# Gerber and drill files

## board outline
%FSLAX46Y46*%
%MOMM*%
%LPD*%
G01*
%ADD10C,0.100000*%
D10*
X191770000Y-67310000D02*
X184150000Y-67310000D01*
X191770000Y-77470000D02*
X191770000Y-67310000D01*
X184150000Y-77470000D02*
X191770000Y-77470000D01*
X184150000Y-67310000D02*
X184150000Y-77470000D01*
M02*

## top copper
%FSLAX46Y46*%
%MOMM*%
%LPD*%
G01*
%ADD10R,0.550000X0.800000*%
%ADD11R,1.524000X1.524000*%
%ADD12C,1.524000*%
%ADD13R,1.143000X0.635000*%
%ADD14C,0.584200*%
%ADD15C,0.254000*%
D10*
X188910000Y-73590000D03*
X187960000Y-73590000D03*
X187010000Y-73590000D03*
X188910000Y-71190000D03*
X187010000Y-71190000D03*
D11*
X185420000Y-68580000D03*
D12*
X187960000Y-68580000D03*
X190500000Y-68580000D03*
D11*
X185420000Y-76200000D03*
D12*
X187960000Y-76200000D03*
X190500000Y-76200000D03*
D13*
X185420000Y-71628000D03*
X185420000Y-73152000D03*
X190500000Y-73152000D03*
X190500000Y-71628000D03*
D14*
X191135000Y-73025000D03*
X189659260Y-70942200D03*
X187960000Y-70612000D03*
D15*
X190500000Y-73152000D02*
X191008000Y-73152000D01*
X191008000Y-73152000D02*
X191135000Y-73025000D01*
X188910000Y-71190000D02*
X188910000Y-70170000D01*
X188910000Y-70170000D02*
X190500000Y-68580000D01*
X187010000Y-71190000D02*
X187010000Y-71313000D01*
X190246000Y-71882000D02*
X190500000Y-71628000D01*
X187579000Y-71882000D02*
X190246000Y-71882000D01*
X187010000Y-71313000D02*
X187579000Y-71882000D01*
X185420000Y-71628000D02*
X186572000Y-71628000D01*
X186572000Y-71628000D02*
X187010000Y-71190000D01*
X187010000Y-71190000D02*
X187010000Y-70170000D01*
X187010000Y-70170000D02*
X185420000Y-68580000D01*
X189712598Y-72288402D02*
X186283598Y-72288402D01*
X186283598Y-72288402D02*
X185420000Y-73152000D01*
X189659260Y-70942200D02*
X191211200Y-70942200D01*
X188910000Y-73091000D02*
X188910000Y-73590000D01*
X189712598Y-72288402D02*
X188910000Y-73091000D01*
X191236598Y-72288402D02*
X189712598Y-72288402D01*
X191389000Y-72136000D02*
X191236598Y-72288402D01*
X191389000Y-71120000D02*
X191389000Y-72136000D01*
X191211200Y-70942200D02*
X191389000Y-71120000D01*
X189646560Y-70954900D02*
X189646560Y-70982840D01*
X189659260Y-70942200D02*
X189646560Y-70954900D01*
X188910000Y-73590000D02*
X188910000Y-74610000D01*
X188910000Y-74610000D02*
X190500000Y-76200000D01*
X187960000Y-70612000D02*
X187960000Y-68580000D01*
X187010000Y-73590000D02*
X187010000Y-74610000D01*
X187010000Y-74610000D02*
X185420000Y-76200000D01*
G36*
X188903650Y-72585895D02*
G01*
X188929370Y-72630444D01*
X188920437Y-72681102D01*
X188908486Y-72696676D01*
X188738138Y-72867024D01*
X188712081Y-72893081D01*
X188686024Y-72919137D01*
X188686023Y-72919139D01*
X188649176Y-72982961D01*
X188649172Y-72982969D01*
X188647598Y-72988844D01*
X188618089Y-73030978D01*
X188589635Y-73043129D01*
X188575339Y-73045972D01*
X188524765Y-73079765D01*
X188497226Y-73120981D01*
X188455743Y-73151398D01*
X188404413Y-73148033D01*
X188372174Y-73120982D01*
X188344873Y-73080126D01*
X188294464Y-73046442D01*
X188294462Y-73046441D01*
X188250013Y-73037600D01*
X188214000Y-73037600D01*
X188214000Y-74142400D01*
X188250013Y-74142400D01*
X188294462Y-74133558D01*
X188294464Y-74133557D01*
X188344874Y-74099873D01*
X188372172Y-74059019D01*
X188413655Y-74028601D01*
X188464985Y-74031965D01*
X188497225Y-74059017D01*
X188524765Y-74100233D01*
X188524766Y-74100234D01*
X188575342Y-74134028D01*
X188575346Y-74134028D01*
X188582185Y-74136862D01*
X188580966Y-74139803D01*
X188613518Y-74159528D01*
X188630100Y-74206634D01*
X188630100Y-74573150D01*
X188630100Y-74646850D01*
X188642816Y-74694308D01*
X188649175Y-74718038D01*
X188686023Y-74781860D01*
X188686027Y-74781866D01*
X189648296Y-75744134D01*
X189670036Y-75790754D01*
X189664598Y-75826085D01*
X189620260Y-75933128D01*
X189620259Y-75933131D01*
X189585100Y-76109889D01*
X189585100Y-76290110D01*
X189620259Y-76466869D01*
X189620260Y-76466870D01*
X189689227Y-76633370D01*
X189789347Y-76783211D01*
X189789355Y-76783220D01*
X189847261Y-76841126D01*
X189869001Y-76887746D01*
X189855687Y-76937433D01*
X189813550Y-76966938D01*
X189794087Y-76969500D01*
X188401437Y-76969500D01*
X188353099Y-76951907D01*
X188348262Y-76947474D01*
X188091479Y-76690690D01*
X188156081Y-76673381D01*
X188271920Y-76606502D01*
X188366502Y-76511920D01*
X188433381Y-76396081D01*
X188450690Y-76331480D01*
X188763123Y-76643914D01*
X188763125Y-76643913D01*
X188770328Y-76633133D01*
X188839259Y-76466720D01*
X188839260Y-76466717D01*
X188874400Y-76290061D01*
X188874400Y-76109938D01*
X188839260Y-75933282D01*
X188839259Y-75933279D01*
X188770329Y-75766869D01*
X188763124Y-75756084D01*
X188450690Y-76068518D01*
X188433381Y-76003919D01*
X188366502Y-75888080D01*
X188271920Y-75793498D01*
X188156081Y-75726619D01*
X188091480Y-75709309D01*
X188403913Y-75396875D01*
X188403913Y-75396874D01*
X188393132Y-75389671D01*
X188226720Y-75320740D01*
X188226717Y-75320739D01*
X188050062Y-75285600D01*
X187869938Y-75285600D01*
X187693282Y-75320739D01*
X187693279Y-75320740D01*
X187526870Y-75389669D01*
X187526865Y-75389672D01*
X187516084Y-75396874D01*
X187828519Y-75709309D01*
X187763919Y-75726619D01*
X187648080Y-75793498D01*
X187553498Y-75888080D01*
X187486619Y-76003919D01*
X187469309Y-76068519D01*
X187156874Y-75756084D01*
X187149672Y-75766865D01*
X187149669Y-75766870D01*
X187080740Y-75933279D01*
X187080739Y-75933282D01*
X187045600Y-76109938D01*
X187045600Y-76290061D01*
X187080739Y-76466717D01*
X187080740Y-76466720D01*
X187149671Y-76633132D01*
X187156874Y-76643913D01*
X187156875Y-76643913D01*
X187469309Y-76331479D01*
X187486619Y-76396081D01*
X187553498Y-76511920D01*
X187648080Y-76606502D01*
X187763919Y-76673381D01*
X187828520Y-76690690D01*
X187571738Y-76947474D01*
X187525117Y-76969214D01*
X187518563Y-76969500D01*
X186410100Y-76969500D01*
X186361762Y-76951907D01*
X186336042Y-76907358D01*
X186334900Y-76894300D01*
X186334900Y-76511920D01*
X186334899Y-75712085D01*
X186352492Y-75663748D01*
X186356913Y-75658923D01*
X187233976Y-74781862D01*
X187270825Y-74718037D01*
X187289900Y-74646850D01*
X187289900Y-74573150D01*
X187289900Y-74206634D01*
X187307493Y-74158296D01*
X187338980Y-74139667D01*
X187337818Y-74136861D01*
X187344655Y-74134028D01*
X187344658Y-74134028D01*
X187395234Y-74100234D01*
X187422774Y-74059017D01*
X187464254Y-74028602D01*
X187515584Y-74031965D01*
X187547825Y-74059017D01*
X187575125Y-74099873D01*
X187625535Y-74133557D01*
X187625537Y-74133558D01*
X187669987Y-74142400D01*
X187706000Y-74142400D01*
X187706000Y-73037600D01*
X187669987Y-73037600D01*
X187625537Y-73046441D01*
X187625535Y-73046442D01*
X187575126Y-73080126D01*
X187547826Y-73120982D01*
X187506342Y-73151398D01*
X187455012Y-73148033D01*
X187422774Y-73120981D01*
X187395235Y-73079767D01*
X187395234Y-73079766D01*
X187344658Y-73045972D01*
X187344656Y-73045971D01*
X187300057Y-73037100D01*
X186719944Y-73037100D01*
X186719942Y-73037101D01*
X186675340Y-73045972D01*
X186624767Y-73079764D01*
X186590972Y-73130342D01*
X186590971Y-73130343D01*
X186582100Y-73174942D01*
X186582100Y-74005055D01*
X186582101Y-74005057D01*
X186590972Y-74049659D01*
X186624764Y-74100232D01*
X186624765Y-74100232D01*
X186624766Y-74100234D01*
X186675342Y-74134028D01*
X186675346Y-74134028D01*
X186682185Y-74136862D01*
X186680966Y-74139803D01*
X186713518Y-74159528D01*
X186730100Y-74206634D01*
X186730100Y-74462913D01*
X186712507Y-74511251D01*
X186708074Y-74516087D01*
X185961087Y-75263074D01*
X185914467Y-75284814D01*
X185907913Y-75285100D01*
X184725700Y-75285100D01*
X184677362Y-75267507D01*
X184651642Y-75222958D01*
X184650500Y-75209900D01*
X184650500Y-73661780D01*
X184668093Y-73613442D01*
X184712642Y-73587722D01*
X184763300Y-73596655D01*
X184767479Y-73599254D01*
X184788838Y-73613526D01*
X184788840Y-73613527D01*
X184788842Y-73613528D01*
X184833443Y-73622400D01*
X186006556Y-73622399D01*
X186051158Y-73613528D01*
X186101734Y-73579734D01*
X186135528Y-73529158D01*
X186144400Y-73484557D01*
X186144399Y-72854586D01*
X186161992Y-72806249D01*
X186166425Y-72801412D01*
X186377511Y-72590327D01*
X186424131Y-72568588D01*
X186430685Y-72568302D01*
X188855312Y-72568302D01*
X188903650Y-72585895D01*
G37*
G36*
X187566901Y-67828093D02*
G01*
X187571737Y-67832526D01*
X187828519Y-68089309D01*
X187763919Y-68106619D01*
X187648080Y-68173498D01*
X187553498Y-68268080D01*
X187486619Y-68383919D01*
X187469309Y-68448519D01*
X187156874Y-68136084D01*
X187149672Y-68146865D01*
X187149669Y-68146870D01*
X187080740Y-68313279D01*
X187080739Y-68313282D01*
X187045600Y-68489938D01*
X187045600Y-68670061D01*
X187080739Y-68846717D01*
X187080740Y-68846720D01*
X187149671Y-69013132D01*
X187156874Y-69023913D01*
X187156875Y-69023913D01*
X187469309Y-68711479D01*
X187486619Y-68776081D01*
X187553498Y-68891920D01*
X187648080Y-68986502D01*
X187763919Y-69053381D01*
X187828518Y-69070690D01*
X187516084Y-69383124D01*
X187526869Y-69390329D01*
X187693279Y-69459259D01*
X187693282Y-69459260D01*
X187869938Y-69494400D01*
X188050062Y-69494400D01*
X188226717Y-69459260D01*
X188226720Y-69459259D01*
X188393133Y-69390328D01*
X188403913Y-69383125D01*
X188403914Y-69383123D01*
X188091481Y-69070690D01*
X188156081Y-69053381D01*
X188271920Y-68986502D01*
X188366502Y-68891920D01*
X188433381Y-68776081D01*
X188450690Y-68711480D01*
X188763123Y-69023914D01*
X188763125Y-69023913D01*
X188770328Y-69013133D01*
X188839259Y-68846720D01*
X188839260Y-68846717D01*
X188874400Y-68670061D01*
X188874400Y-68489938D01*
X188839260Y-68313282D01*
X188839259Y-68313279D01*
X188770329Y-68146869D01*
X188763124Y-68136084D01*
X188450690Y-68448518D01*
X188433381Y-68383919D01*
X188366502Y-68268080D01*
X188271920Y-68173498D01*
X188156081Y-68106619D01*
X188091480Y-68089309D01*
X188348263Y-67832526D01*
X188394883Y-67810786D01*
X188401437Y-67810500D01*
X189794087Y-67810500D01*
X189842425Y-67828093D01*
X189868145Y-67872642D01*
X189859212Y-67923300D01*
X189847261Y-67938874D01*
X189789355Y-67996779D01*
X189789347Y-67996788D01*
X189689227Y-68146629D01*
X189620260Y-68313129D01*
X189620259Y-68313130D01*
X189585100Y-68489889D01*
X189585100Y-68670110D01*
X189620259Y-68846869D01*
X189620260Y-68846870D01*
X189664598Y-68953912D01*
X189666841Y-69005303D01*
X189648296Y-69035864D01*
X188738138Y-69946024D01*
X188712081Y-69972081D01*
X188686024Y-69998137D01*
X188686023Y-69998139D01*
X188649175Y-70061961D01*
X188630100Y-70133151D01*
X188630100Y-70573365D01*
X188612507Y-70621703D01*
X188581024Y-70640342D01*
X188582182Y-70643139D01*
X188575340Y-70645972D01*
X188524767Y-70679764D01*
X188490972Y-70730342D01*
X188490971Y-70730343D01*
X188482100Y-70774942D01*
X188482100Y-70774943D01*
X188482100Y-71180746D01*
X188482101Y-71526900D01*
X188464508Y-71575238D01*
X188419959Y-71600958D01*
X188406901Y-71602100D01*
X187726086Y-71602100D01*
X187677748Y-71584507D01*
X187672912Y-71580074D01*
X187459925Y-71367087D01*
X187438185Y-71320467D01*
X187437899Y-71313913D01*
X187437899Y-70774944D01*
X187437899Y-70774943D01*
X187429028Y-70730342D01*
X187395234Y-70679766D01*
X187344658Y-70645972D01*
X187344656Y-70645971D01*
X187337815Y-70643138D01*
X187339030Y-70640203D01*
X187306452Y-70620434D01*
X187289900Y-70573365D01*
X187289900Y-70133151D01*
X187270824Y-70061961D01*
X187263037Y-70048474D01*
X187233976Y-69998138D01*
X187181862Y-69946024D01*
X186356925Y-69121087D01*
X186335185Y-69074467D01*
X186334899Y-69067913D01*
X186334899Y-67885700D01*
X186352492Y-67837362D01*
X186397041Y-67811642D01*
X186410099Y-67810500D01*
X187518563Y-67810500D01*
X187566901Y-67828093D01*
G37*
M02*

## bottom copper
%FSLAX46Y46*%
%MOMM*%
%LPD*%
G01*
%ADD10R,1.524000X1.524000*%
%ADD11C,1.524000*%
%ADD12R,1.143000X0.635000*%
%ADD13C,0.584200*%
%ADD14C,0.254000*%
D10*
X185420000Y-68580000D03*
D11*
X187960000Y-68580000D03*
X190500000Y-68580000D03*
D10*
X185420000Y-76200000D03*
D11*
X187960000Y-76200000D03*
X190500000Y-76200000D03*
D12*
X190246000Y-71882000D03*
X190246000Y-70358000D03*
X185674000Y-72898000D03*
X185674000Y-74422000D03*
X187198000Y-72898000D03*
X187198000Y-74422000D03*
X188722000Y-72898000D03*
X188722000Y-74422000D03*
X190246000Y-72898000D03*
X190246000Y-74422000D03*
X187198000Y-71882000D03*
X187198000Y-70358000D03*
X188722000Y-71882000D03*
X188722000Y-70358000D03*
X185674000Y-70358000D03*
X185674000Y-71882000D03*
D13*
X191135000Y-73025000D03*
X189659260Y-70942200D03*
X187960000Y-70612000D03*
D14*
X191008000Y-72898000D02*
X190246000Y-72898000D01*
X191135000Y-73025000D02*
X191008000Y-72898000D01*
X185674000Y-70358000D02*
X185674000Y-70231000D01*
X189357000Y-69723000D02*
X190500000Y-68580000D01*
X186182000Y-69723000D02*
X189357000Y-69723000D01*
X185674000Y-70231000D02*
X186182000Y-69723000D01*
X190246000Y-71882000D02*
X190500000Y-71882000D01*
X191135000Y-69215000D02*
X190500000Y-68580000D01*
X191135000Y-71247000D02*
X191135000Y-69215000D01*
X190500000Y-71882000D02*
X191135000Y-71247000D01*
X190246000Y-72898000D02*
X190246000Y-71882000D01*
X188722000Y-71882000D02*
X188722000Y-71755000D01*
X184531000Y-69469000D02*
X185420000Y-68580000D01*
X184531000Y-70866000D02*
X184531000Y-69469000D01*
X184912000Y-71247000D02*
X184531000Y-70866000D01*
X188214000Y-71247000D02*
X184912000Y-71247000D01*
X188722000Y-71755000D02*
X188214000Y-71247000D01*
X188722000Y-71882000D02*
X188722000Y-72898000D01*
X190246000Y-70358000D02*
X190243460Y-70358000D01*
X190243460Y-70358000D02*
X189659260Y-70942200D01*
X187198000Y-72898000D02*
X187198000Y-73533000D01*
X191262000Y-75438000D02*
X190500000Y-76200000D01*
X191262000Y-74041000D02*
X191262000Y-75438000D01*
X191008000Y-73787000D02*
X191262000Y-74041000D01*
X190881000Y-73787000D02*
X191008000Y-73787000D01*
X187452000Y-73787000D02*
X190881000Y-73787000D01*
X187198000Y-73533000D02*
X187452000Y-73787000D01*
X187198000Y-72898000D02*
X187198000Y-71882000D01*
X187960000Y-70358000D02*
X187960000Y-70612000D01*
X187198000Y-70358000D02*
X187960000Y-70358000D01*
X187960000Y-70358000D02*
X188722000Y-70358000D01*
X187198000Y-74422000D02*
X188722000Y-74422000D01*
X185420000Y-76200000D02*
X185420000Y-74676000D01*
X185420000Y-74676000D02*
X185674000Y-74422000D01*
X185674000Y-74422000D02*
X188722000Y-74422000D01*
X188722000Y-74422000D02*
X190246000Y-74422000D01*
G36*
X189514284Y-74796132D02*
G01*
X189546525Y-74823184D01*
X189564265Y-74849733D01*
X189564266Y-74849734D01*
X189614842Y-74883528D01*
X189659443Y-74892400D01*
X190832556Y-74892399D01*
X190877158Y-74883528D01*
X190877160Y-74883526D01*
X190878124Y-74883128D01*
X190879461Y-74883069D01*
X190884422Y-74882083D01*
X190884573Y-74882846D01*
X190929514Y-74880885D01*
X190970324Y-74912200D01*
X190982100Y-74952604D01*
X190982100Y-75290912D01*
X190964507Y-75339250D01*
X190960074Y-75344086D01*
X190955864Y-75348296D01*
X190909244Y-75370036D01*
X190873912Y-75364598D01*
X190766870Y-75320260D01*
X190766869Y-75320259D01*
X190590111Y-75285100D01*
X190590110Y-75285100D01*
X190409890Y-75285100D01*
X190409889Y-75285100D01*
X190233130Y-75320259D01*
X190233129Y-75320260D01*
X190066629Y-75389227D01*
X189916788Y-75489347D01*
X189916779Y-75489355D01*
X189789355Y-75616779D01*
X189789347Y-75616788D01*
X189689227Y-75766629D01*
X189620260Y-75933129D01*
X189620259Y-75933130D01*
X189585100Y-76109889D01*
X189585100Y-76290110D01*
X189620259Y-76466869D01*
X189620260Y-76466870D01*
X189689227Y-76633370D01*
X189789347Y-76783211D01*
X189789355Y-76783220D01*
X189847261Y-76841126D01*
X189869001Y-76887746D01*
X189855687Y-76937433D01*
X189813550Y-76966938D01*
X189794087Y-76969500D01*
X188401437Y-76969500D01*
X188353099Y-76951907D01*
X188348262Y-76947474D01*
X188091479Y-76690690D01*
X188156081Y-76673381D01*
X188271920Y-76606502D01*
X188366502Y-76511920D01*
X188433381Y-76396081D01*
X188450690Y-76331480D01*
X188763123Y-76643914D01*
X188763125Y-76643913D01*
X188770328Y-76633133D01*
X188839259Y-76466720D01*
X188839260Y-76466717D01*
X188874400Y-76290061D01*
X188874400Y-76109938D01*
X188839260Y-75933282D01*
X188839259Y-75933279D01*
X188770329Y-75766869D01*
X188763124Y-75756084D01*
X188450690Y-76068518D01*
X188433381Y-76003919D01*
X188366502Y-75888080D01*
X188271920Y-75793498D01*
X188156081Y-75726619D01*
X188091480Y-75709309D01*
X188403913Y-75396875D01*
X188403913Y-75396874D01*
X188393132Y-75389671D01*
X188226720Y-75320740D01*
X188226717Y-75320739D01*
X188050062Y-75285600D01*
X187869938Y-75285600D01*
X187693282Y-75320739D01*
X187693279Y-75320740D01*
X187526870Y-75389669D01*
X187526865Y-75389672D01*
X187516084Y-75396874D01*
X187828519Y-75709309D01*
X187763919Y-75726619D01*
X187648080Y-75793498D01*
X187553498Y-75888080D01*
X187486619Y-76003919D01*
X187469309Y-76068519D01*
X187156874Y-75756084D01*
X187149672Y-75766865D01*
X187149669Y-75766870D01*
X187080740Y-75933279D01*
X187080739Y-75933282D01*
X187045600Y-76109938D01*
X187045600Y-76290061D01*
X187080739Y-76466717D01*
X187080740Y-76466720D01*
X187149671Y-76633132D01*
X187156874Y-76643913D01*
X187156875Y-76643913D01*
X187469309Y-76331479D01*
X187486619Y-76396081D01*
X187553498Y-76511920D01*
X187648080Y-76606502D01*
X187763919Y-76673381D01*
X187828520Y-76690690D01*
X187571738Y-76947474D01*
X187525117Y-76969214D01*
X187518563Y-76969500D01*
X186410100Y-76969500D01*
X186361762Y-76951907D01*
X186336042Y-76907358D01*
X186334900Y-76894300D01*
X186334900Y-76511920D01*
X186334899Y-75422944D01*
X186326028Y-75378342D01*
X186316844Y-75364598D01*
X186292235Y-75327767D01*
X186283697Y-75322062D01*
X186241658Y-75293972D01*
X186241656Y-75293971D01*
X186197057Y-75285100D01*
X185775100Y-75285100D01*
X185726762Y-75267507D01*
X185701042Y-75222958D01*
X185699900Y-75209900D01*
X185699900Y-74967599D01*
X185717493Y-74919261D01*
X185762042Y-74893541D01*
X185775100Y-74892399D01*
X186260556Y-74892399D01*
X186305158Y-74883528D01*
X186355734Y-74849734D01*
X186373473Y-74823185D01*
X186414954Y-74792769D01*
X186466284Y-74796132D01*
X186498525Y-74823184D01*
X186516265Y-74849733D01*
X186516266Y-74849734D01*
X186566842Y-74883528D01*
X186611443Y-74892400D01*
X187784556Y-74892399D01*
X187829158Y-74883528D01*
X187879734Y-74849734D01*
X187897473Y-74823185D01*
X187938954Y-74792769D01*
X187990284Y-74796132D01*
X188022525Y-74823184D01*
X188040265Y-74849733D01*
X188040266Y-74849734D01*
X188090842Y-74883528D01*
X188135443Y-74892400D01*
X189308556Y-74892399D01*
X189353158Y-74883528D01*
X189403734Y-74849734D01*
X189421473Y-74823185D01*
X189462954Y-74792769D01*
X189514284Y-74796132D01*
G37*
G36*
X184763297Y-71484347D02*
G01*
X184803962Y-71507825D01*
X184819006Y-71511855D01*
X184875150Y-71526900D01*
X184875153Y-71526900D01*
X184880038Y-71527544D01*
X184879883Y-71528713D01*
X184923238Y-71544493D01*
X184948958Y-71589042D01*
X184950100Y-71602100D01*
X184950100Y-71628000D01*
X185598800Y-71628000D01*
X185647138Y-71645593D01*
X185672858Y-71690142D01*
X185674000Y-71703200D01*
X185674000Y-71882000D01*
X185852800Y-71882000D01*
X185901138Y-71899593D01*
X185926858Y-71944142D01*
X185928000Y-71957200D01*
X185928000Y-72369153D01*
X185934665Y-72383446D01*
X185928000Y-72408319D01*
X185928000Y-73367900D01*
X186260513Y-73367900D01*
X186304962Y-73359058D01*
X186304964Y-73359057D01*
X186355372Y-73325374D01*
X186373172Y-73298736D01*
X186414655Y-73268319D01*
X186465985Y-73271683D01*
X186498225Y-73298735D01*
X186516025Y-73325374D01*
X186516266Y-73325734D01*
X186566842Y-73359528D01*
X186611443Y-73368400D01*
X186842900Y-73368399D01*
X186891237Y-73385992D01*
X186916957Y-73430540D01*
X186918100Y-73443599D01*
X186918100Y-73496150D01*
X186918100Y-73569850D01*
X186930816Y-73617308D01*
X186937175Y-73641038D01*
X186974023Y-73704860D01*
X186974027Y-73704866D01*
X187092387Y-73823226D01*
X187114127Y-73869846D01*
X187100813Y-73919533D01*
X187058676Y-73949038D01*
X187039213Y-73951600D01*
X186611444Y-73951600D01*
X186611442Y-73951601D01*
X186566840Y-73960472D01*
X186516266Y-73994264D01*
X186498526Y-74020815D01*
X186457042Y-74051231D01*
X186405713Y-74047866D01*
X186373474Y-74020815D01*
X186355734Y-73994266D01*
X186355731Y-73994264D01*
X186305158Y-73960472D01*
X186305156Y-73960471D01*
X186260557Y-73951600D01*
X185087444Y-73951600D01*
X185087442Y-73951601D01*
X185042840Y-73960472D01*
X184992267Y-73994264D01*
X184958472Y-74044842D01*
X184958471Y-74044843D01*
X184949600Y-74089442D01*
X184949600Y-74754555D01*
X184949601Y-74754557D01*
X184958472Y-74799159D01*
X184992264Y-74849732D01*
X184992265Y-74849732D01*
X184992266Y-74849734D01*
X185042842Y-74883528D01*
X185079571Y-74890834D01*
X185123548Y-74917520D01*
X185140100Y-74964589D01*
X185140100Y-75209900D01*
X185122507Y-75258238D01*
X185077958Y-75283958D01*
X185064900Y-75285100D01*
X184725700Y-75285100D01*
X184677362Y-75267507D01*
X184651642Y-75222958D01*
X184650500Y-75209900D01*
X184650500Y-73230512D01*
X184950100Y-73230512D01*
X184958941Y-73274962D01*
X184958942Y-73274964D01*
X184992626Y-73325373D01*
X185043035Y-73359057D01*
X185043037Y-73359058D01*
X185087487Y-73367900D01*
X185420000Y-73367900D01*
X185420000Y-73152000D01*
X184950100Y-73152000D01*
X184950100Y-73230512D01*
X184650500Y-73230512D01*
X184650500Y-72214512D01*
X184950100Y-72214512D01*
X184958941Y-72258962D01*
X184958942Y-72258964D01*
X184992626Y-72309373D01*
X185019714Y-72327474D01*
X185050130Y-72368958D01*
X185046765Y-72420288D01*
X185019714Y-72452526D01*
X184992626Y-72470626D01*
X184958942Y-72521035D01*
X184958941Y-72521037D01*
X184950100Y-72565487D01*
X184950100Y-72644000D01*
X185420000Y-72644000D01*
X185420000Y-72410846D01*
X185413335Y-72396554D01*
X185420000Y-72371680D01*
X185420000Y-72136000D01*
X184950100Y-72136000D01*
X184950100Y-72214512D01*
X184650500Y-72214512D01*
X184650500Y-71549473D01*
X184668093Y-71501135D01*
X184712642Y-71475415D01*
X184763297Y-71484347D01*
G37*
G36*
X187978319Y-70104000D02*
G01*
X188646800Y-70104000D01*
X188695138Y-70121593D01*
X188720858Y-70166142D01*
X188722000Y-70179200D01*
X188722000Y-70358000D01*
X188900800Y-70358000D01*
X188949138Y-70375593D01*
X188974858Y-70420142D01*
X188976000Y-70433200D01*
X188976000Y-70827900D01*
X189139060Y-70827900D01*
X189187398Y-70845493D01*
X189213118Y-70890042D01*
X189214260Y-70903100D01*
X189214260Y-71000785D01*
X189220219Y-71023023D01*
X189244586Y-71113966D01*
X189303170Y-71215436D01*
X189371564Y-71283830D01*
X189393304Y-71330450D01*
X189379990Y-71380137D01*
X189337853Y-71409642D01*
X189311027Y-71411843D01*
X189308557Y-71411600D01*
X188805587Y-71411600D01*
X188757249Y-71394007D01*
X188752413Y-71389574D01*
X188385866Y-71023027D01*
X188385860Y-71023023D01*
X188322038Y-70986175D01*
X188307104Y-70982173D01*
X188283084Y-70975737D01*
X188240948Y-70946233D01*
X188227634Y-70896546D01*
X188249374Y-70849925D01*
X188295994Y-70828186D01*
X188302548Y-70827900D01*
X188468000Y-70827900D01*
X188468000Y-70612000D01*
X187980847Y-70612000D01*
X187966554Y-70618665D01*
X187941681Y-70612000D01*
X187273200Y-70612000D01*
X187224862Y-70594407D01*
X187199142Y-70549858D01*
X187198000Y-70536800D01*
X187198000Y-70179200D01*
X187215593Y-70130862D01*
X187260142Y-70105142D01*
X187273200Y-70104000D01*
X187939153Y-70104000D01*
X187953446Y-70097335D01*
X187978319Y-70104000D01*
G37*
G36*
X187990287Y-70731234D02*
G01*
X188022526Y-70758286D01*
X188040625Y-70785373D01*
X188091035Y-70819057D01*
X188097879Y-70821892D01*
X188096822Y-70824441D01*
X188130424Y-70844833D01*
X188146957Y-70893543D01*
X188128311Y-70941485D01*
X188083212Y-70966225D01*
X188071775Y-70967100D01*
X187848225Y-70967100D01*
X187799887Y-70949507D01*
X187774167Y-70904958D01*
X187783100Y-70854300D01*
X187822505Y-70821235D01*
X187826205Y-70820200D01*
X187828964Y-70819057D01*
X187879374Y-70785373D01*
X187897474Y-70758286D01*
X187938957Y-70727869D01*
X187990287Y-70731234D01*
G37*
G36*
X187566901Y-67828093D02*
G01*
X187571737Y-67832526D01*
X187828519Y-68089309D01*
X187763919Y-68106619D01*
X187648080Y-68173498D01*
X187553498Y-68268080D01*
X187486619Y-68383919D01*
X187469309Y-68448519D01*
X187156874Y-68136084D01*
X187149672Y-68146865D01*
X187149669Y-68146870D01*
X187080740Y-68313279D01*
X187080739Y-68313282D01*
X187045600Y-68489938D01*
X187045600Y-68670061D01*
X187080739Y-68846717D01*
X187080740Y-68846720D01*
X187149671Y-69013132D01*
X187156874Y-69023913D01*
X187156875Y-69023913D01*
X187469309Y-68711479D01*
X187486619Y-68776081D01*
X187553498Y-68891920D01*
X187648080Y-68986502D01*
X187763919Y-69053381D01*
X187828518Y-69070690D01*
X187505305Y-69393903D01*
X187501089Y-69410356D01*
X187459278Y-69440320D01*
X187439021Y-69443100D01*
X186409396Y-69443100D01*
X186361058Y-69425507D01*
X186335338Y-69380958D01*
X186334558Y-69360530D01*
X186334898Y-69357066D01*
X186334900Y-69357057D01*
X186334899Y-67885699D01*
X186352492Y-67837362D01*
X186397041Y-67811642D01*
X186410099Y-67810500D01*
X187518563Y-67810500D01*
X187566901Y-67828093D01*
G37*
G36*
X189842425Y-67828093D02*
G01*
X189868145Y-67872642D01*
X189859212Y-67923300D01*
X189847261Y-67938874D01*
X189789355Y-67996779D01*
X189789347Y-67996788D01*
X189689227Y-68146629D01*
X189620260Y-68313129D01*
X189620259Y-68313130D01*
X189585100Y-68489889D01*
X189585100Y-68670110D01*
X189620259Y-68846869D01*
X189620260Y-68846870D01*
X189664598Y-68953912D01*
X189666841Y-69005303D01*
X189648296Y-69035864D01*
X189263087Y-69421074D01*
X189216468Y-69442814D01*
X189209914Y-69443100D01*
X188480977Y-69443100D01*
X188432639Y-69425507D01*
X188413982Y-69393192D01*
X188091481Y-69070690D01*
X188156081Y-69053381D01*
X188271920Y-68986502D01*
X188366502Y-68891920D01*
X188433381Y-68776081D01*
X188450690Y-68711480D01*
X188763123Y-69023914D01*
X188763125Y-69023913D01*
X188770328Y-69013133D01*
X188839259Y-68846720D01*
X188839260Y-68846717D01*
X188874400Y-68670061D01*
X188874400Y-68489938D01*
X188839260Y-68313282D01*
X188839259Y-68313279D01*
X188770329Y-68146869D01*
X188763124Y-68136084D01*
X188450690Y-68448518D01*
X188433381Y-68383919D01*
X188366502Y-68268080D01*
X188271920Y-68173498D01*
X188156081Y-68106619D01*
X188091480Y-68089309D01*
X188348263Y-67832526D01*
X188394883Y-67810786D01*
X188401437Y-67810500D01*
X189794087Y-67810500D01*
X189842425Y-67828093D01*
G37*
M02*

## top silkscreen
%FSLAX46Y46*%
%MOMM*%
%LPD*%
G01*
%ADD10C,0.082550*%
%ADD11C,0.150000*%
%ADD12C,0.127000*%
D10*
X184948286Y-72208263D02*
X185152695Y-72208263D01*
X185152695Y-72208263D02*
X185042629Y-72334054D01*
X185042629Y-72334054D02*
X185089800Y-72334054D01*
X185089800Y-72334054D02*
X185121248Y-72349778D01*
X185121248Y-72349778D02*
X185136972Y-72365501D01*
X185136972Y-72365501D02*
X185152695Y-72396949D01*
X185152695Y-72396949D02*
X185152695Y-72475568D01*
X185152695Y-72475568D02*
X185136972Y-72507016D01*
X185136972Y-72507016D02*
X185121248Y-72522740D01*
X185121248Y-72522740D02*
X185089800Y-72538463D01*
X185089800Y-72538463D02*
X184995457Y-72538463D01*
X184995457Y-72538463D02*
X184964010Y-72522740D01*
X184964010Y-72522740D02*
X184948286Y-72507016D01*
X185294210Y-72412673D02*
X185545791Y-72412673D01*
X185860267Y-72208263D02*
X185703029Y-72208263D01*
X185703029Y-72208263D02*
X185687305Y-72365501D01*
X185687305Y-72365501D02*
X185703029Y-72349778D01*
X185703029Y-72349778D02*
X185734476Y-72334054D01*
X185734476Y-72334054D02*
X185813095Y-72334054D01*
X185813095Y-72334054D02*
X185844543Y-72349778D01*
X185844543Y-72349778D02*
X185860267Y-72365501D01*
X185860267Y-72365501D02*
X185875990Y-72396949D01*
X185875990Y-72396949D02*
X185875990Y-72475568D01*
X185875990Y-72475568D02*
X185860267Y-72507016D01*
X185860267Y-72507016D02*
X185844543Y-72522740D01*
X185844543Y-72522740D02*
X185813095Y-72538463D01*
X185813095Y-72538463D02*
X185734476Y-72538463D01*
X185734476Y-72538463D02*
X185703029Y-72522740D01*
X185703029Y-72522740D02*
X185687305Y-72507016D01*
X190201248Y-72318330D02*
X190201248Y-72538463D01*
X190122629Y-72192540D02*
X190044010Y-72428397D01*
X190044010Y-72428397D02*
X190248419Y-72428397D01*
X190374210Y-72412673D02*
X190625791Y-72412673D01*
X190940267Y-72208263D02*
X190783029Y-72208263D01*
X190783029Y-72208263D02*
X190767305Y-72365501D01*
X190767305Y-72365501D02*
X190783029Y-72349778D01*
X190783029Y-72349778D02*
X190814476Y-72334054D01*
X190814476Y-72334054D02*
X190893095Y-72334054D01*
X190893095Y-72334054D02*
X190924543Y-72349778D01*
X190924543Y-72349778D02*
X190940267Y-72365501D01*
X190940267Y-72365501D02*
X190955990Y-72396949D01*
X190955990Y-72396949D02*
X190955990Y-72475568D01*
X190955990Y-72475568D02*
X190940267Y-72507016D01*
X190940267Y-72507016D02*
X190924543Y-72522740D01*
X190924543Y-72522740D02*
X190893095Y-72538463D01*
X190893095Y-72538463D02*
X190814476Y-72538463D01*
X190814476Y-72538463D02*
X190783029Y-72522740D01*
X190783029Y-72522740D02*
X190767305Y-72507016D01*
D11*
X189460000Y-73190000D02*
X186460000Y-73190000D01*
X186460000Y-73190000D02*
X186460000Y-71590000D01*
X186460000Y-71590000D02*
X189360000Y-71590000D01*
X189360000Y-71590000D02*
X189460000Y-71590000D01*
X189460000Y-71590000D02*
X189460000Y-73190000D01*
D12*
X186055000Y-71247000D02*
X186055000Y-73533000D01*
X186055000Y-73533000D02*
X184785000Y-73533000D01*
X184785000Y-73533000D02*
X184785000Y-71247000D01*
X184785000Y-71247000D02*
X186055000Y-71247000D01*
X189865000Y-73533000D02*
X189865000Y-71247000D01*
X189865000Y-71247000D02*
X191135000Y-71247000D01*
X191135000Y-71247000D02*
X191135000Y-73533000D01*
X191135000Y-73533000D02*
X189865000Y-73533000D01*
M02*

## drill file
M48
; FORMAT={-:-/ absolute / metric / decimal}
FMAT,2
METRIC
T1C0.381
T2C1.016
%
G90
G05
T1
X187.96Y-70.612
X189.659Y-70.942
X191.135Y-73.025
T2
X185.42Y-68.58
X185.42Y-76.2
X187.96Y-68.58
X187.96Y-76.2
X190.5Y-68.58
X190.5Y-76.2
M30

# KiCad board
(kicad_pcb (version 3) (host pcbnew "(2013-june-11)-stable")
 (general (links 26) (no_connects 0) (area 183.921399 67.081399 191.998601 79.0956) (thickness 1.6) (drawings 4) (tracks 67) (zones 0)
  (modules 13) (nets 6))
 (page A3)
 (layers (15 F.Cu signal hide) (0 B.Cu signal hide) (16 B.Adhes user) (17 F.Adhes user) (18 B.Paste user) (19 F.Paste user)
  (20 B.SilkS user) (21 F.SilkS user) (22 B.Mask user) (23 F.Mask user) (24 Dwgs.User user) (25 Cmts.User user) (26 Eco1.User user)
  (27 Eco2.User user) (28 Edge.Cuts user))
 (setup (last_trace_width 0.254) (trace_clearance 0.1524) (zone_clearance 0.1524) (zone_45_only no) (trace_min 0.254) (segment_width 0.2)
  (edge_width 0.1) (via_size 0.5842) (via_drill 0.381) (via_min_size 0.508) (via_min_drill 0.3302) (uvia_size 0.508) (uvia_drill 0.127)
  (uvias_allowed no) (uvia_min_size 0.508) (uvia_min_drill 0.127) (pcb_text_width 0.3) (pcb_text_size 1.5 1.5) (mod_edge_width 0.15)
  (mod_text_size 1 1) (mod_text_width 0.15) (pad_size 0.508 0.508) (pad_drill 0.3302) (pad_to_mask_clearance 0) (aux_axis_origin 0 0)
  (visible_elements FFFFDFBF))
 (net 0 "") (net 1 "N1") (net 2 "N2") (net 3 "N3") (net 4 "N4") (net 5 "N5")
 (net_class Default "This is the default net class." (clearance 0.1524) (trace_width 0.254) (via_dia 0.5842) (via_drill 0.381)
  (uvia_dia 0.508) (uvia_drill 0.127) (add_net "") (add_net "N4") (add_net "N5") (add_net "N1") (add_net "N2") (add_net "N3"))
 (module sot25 (layer F.Cu) (at 187.96 72.39 180)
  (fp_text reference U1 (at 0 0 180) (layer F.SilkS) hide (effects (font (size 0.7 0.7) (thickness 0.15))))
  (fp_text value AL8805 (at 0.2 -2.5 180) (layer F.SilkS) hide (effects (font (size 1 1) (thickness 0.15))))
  (fp_line (start -1.5 -0.8) (end 1.5 -0.8) (layer F.SilkS) (width 0.15))
  (fp_line (start 1.5 -0.8) (end 1.5 0.8) (layer F.SilkS) (width 0.15))
  (fp_line (start 1.5 0.8) (end -1.4 0.8) (layer F.SilkS) (width 0.15))
  (fp_line (start -1.4 0.8) (end -1.5 0.8) (layer F.SilkS) (width 0.15))
  (fp_line (start -1.5 0.8) (end -1.5 -0.8) (layer F.SilkS) (width 0.15))
  (pad 3 smd rect (at -0.95 -1.2 180) (size 0.55 0.8) (layers F.Cu F.Paste F.Mask) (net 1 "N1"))
  (pad 2 smd rect (at 0 -1.2 180) (size 0.55 0.8) (layers F.Cu F.Paste F.Mask) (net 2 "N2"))
  (pad 1 smd rect (at 0.95 -1.2 180) (size 0.55 0.8) (layers F.Cu F.Paste F.Mask) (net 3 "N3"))
  (pad 4 smd rect (at -0.95 1.2 180) (size 0.55 0.8) (layers F.Cu F.Paste F.Mask) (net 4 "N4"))
  (pad 5 smd rect (at 0.95 1.2 180) (size 0.55 0.8) (layers F.Cu F.Paste F.Mask) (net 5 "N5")))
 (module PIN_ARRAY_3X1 (layer B.Cu) (at 187.96 68.58)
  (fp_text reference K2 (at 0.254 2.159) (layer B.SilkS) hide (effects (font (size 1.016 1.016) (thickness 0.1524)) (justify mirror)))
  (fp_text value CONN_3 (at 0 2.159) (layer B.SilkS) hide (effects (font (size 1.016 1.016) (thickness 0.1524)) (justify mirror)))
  (pad 1 thru_hole rect (at -2.54 0) (size 1.524 1.524) (drill 1.016) (layers *.Cu *.Mask B.SilkS) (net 5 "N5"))
  (pad 2 thru_hole circle (at 0 0) (size 1.524 1.524) (drill 1.016) (layers *.Cu *.Mask B.SilkS) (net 2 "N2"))
  (pad 3 thru_hole circle (at 2.54 0) (size 1.524 1.524) (drill 1.016) (layers *.Cu *.Mask B.SilkS) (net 4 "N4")))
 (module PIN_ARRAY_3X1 (layer B.Cu) (at 187.96 76.2)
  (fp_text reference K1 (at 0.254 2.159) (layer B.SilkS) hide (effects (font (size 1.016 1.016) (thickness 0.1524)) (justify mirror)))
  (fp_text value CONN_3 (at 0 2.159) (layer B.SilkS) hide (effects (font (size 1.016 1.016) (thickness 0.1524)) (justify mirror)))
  (pad 1 thru_hole rect (at -2.54 0) (size 1.524 1.524) (drill 1.016) (layers *.Cu *.Mask B.SilkS) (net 3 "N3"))
  (pad 2 thru_hole circle (at 0 0) (size 1.524 1.524) (drill 1.016) (layers *.Cu *.Mask B.SilkS) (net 2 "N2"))
  (pad 3 thru_hole circle (at 2.54 0) (size 1.524 1.524) (drill 1.016) (layers *.Cu *.Mask B.SilkS) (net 1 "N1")))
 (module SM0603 (layer F.Cu) (at 185.42 72.39 270)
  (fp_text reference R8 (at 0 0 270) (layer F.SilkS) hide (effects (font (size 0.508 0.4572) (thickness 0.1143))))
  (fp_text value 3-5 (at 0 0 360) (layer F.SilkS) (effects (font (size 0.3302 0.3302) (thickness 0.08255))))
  (fp_line (start -1.143 -0.635) (end 1.143 -0.635) (layer F.SilkS) (width 0.127))
  (fp_line (start 1.143 -0.635) (end 1.143 0.635) (layer F.SilkS) (width 0.127))
  (fp_line (start 1.143 0.635) (end -1.143 0.635) (layer F.SilkS) (width 0.127))
  (fp_line (start -1.143 0.635) (end -1.143 -0.635) (layer F.SilkS) (width 0.127))
  (pad 1 smd rect (at -0.762 0 270) (size 0.635 1.143) (layers F.Cu F.Paste F.Mask) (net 5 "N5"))
  (pad 2 smd rect (at 0.762 0 270) (size 0.635 1.143) (layers F.Cu F.Paste F.Mask) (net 1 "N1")))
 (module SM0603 (layer B.Cu) (at 190.246 71.12 90)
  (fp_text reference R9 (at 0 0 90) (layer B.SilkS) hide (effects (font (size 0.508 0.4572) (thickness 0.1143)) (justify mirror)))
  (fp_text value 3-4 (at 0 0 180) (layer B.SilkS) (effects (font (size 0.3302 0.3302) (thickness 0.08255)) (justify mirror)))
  (pad 1 smd rect (at -0.762 0 90) (size 0.635 1.143) (layers B.Cu B.Paste B.Mask) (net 4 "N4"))
  (pad 2 smd rect (at 0.762 0 90) (size 0.635 1.143) (layers B.Cu B.Paste B.Mask) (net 1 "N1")))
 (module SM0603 (layer F.Cu) (at 190.5 72.39 90)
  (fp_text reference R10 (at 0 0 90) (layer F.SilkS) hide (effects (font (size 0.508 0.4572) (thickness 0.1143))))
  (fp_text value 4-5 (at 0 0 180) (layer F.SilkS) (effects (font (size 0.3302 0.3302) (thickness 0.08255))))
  (fp_line (start -1.143 -0.635) (end 1.143 -0.635) (layer F.SilkS) (width 0.127))
  (fp_line (start 1.143 -0.635) (end 1.143 0.635) (layer F.SilkS) (width 0.127))
  (fp_line (start 1.143 0.635) (end -1.143 0.635) (layer F.SilkS) (width 0.127))
  (fp_line (start -1.143 0.635) (end -1.143 -0.635) (layer F.SilkS) (width 0.127))
  (pad 1 smd rect (at -0.762 0 90) (size 0.635 1.143) (layers F.Cu F.Paste F.Mask) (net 4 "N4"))
  (pad 2 smd rect (at 0.762 0 90) (size 0.635 1.143) (layers F.Cu F.Paste F.Mask) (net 5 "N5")))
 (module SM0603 (layer B.Cu) (at 185.674 73.66 270)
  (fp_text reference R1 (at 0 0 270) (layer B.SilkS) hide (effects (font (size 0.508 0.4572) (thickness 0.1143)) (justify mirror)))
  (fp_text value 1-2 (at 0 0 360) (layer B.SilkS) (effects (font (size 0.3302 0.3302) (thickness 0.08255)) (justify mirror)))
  (pad 1 smd rect (at -0.762 0 270) (size 0.635 1.143) (layers B.Cu B.Paste B.Mask) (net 2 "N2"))
  (pad 2 smd rect (at 0.762 0 270) (size 0.635 1.143) (layers B.Cu B.Paste B.Mask) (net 3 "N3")))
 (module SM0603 (layer B.Cu) (at 187.198 73.66 270)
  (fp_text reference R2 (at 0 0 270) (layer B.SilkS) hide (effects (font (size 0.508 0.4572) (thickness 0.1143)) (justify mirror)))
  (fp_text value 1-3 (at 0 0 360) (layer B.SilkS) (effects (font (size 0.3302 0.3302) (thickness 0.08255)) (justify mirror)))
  (pad 1 smd rect (at -0.762 0 270) (size 0.635 1.143) (layers B.Cu B.Paste B.Mask) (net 1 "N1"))
  (pad 2 smd rect (at 0.762 0 270) (size 0.635 1.143) (layers B.Cu B.Paste B.Mask) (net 3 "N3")))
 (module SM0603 (layer B.Cu) (at 188.722 73.66 270)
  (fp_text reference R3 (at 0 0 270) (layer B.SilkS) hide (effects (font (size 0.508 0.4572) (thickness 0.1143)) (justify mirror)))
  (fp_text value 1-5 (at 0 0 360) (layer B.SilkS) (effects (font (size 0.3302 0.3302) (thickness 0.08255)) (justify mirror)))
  (pad 1 smd rect (at -0.762 0 270) (size 0.635 1.143) (layers B.Cu B.Paste B.Mask) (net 5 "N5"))
  (pad 2 smd rect (at 0.762 0 270) (size 0.635 1.143) (layers B.Cu B.Paste B.Mask) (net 3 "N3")))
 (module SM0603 (layer B.Cu) (at 190.246 73.66 270)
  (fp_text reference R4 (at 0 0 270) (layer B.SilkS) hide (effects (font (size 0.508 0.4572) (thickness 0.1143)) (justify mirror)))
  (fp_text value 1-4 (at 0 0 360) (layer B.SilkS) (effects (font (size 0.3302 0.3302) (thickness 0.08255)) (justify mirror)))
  (pad 1 smd rect (at -0.762 0 270) (size 0.635 1.143) (layers B.Cu B.Paste B.Mask) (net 4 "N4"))
  (pad 2 smd rect (at 0.762 0 270) (size 0.635 1.143) (layers B.Cu B.Paste B.Mask) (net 3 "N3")))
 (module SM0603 (layer B.Cu) (at 187.198 71.12 90)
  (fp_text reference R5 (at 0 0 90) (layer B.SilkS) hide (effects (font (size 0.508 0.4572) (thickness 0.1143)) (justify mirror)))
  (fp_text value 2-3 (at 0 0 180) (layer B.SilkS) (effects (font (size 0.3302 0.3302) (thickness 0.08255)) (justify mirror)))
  (pad 1 smd rect (at -0.762 0 90) (size 0.635 1.143) (layers B.Cu B.Paste B.Mask) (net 1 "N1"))
  (pad 2 smd rect (at 0.762 0 90) (size 0.635 1.143) (layers B.Cu B.Paste B.Mask) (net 2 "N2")))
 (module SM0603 (layer B.Cu) (at 188.722 71.12 90)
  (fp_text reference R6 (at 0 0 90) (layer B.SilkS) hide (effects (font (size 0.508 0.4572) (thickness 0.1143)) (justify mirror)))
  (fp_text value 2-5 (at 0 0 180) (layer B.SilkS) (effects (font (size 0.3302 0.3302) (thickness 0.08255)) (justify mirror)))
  (pad 1 smd rect (at -0.762 0 90) (size 0.635 1.143) (layers B.Cu B.Paste B.Mask) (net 5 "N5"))
  (pad 2 smd rect (at 0.762 0 90) (size 0.635 1.143) (layers B.Cu B.Paste B.Mask) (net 2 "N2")))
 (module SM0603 (layer B.Cu) (at 185.674 71.12 270)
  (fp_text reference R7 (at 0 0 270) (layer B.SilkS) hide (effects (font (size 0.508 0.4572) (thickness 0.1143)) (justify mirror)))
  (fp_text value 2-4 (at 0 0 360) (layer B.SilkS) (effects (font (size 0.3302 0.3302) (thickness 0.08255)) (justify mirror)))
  (pad 1 smd rect (at -0.762 0 270) (size 0.635 1.143) (layers B.Cu B.Paste B.Mask) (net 4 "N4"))
  (pad 2 smd rect (at 0.762 0 270) (size 0.635 1.143) (layers B.Cu B.Paste B.Mask) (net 2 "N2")))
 (gr_line (start 191.77 67.31) (end 184.15 67.31) (angle 90) (layer Edge.Cuts) (width 0.1))
 (gr_line (start 191.77 77.47) (end 191.77 67.31) (angle 90) (layer Edge.Cuts) (width 0.1))
 (gr_line (start 184.15 77.47) (end 191.77 77.47) (angle 90) (layer Edge.Cuts) (width 0.1))
 (gr_line (start 184.15 67.31) (end 184.15 77.47) (angle 90) (layer Edge.Cuts) (width 0.1))
 (segment (start 190.5 73.152) (end 191.008 73.152) (width 0.254) (layer F.Cu) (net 4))
 (segment (start 191.008 72.898) (end 190.246 72.898) (width 0.254) (layer B.Cu) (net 4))
 (segment (start 191.135 73.025) (end 191.008 72.898) (width 0.254) (layer B.Cu) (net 4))
 (via (at 191.135 73.025) (size 0.5842) (layers F.Cu B.Cu) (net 4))
 (segment (start 191.008 73.152) (end 191.135 73.025) (width 0.254) (layer F.Cu) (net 4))
 (segment (start 185.674 70.358) (end 185.674 70.231) (width 0.254) (layer B.Cu) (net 4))
 (segment (start 189.357 69.723) (end 190.5 68.58) (width 0.254) (layer B.Cu) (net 4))
 (segment (start 186.182 69.723) (end 189.357 69.723) (width 0.254) (layer B.Cu) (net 4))
 (segment (start 185.674 70.231) (end 186.182 69.723) (width 0.254) (layer B.Cu) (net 4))
 (segment (start 190.246 71.882) (end 190.5 71.882) (width 0.254) (layer B.Cu) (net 4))
 (segment (start 191.135 69.215) (end 190.5 68.58) (width 0.254) (layer B.Cu) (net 4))
 (segment (start 191.135 71.247) (end 191.135 69.215) (width 0.254) (layer B.Cu) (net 4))
 (segment (start 190.5 71.882) (end 191.135 71.247) (width 0.254) (layer B.Cu) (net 4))
 (segment (start 190.246 72.898) (end 190.246 71.882) (width 0.254) (layer B.Cu) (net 4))
 (segment (start 188.91 71.19) (end 188.91 70.17) (width 0.254) (layer F.Cu) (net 4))
 (segment (start 188.91 70.17) (end 190.5 68.58) (width 0.254) (layer F.Cu) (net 4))
 (segment (start 187.01 71.19) (end 187.01 71.313) (width 0.254) (layer F.Cu) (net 5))
 (segment (start 190.246 71.882) (end 190.5 71.628) (width 0.254) (layer F.Cu) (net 5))
 (segment (start 187.579 71.882) (end 190.246 71.882) (width 0.254) (layer F.Cu) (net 5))
 (segment (start 187.01 71.313) (end 187.579 71.882) (width 0.254) (layer F.Cu) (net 5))
 (segment (start 185.42 71.628) (end 186.572 71.628) (width 0.254) (layer F.Cu) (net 5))
 (segment (start 186.572 71.628) (end 187.01 71.19) (width 0.254) (layer F.Cu) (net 5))
 (segment (start 188.722 71.882) (end 188.722 71.755) (width 0.254) (layer B.Cu) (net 5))
 (segment (start 184.531 69.469) (end 185.42 68.58) (width 0.254) (layer B.Cu) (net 5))
 (segment (start 184.531 70.866) (end 184.531 69.469) (width 0.254) (layer B.Cu) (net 5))
 (segment (start 184.912 71.247) (end 184.531 70.866) (width 0.254) (layer B.Cu) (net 5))
 (segment (start 188.214 71.247) (end 184.912 71.247) (width 0.254) (layer B.Cu) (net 5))
 (segment (start 188.722 71.755) (end 188.214 71.247) (width 0.254) (layer B.Cu) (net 5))
 (segment (start 188.722 71.882) (end 188.722 72.898) (width 0.254) (layer B.Cu) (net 5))
 (segment (start 187.01 71.19) (end 187.01 70.17) (width 0.254) (layer F.Cu) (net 5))
 (segment (start 187.01 70.17) (end 185.42 68.58) (width 0.254) (layer F.Cu) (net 5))
 (segment (start 189.712598 72.288402) (end 186.283598 72.288402) (width 0.254) (layer F.Cu) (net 1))
 (segment (start 186.283598 72.288402) (end 185.42 73.152) (width 0.254) (layer F.Cu) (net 1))
 (segment (start 189.65926 70.9422) (end 191.2112 70.9422) (width 0.254) (layer F.Cu) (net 1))
 (segment (start 188.91 73.091) (end 188.91 73.59) (width 0.254) (layer F.Cu) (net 1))
 (segment (start 189.712598 72.288402) (end 188.91 73.091) (width 0.254) (layer F.Cu) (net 1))
 (segment (start 191.236598 72.288402) (end 189.712598 72.288402) (width 0.254) (layer F.Cu) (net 1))
 (segment (start 191.389 72.136) (end 191.236598 72.288402) (width 0.254) (layer F.Cu) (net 1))
 (segment (start 191.389 71.12) (end 191.389 72.136) (width 0.254) (layer F.Cu) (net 1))
 (segment (start 191.2112 70.9422) (end 191.389 71.12) (width 0.254) (layer F.Cu) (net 1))
 (segment (start 190.246 70.358) (end 190.24346 70.358) (width 0.254) (layer B.Cu) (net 1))
 (segment (start 189.64656 70.9549) (end 189.64656 70.98284) (width 0.254) (layer F.Cu) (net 1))
 (segment (start 189.65926 70.9422) (end 189.64656 70.9549) (width 0.254) (layer F.Cu) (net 1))
 (via (at 189.65926 70.9422) (size 0.5842) (layers F.Cu B.Cu) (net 1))
 (segment (start 190.24346 70.358) (end 189.65926 70.9422) (width 0.254) (layer B.Cu) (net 1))
 (segment (start 187.198 72.898) (end 187.198 73.533) (width 0.254) (layer B.Cu) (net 1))
 (segment (start 191.262 75.438) (end 190.5 76.2) (width 0.254) (layer B.Cu) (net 1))
 (segment (start 191.262 74.041) (end 191.262 75.438) (width 0.254) (layer B.Cu) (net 1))
 (segment (start 191.008 73.787) (end 191.262 74.041) (width 0.254) (layer B.Cu) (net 1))
 (segment (start 190.881 73.787) (end 191.008 73.787) (width 0.254) (layer B.Cu) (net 1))
 (segment (start 187.452 73.787) (end 190.881 73.787) (width 0.254) (layer B.Cu) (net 1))
 (segment (start 187.198 73.533) (end 187.452 73.787) (width 0.254) (layer B.Cu) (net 1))
 (segment (start 187.198 72.898) (end 187.198 71.882) (width 0.254) (layer B.Cu) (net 1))
 (segment (start 188.91 73.59) (end 188.91 74.61) (width 0.254) (layer F.Cu) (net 1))
 (segment (start 188.91 74.61) (end 190.5 76.2) (width 0.254) (layer F.Cu) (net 1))
 (segment (start 187.96 70.358) (end 187.96 70.612) (width 0.254) (layer B.Cu) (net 2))
 (segment (start 187.96 70.612) (end 187.96 68.58) (width 0.254) (layer F.Cu) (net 2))
 (via (at 187.96 70.612) (size 0.5842) (layers F.Cu B.Cu) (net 2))
 (segment (start 187.198 70.358) (end 187.96 70.358) (width 0.254) (layer B.Cu) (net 2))
 (segment (start 187.96 70.358) (end 188.722 70.358) (width 0.254) (layer B.Cu) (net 2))
 (segment (start 187.198 74.422) (end 188.722 74.422) (width 0.254) (layer B.Cu) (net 3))
 (segment (start 185.42 76.2) (end 185.42 74.676) (width 0.254) (layer B.Cu) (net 3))
 (segment (start 185.42 74.676) (end 185.674 74.422) (width 0.254) (layer B.Cu) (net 3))
 (segment (start 185.674 74.422) (end 188.722 74.422) (width 0.254) (layer B.Cu) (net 3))
 (segment (start 188.722 74.422) (end 190.246 74.422) (width 0.254) (layer B.Cu) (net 3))
 (segment (start 187.01 73.59) (end 187.01 74.61) (width 0.254) (layer F.Cu) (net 3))
 (segment (start 187.01 74.61) (end 185.42 76.2) (width 0.254) (layer F.Cu) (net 3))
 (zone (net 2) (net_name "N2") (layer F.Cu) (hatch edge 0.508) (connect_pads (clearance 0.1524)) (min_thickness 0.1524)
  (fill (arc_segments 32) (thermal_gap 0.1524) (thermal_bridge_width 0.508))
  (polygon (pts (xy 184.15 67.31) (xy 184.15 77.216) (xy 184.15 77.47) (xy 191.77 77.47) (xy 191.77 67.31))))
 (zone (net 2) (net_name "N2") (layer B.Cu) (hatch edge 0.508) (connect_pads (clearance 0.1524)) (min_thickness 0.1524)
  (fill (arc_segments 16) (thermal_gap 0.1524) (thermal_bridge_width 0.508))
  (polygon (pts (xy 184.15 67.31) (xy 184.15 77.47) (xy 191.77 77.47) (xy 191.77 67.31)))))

